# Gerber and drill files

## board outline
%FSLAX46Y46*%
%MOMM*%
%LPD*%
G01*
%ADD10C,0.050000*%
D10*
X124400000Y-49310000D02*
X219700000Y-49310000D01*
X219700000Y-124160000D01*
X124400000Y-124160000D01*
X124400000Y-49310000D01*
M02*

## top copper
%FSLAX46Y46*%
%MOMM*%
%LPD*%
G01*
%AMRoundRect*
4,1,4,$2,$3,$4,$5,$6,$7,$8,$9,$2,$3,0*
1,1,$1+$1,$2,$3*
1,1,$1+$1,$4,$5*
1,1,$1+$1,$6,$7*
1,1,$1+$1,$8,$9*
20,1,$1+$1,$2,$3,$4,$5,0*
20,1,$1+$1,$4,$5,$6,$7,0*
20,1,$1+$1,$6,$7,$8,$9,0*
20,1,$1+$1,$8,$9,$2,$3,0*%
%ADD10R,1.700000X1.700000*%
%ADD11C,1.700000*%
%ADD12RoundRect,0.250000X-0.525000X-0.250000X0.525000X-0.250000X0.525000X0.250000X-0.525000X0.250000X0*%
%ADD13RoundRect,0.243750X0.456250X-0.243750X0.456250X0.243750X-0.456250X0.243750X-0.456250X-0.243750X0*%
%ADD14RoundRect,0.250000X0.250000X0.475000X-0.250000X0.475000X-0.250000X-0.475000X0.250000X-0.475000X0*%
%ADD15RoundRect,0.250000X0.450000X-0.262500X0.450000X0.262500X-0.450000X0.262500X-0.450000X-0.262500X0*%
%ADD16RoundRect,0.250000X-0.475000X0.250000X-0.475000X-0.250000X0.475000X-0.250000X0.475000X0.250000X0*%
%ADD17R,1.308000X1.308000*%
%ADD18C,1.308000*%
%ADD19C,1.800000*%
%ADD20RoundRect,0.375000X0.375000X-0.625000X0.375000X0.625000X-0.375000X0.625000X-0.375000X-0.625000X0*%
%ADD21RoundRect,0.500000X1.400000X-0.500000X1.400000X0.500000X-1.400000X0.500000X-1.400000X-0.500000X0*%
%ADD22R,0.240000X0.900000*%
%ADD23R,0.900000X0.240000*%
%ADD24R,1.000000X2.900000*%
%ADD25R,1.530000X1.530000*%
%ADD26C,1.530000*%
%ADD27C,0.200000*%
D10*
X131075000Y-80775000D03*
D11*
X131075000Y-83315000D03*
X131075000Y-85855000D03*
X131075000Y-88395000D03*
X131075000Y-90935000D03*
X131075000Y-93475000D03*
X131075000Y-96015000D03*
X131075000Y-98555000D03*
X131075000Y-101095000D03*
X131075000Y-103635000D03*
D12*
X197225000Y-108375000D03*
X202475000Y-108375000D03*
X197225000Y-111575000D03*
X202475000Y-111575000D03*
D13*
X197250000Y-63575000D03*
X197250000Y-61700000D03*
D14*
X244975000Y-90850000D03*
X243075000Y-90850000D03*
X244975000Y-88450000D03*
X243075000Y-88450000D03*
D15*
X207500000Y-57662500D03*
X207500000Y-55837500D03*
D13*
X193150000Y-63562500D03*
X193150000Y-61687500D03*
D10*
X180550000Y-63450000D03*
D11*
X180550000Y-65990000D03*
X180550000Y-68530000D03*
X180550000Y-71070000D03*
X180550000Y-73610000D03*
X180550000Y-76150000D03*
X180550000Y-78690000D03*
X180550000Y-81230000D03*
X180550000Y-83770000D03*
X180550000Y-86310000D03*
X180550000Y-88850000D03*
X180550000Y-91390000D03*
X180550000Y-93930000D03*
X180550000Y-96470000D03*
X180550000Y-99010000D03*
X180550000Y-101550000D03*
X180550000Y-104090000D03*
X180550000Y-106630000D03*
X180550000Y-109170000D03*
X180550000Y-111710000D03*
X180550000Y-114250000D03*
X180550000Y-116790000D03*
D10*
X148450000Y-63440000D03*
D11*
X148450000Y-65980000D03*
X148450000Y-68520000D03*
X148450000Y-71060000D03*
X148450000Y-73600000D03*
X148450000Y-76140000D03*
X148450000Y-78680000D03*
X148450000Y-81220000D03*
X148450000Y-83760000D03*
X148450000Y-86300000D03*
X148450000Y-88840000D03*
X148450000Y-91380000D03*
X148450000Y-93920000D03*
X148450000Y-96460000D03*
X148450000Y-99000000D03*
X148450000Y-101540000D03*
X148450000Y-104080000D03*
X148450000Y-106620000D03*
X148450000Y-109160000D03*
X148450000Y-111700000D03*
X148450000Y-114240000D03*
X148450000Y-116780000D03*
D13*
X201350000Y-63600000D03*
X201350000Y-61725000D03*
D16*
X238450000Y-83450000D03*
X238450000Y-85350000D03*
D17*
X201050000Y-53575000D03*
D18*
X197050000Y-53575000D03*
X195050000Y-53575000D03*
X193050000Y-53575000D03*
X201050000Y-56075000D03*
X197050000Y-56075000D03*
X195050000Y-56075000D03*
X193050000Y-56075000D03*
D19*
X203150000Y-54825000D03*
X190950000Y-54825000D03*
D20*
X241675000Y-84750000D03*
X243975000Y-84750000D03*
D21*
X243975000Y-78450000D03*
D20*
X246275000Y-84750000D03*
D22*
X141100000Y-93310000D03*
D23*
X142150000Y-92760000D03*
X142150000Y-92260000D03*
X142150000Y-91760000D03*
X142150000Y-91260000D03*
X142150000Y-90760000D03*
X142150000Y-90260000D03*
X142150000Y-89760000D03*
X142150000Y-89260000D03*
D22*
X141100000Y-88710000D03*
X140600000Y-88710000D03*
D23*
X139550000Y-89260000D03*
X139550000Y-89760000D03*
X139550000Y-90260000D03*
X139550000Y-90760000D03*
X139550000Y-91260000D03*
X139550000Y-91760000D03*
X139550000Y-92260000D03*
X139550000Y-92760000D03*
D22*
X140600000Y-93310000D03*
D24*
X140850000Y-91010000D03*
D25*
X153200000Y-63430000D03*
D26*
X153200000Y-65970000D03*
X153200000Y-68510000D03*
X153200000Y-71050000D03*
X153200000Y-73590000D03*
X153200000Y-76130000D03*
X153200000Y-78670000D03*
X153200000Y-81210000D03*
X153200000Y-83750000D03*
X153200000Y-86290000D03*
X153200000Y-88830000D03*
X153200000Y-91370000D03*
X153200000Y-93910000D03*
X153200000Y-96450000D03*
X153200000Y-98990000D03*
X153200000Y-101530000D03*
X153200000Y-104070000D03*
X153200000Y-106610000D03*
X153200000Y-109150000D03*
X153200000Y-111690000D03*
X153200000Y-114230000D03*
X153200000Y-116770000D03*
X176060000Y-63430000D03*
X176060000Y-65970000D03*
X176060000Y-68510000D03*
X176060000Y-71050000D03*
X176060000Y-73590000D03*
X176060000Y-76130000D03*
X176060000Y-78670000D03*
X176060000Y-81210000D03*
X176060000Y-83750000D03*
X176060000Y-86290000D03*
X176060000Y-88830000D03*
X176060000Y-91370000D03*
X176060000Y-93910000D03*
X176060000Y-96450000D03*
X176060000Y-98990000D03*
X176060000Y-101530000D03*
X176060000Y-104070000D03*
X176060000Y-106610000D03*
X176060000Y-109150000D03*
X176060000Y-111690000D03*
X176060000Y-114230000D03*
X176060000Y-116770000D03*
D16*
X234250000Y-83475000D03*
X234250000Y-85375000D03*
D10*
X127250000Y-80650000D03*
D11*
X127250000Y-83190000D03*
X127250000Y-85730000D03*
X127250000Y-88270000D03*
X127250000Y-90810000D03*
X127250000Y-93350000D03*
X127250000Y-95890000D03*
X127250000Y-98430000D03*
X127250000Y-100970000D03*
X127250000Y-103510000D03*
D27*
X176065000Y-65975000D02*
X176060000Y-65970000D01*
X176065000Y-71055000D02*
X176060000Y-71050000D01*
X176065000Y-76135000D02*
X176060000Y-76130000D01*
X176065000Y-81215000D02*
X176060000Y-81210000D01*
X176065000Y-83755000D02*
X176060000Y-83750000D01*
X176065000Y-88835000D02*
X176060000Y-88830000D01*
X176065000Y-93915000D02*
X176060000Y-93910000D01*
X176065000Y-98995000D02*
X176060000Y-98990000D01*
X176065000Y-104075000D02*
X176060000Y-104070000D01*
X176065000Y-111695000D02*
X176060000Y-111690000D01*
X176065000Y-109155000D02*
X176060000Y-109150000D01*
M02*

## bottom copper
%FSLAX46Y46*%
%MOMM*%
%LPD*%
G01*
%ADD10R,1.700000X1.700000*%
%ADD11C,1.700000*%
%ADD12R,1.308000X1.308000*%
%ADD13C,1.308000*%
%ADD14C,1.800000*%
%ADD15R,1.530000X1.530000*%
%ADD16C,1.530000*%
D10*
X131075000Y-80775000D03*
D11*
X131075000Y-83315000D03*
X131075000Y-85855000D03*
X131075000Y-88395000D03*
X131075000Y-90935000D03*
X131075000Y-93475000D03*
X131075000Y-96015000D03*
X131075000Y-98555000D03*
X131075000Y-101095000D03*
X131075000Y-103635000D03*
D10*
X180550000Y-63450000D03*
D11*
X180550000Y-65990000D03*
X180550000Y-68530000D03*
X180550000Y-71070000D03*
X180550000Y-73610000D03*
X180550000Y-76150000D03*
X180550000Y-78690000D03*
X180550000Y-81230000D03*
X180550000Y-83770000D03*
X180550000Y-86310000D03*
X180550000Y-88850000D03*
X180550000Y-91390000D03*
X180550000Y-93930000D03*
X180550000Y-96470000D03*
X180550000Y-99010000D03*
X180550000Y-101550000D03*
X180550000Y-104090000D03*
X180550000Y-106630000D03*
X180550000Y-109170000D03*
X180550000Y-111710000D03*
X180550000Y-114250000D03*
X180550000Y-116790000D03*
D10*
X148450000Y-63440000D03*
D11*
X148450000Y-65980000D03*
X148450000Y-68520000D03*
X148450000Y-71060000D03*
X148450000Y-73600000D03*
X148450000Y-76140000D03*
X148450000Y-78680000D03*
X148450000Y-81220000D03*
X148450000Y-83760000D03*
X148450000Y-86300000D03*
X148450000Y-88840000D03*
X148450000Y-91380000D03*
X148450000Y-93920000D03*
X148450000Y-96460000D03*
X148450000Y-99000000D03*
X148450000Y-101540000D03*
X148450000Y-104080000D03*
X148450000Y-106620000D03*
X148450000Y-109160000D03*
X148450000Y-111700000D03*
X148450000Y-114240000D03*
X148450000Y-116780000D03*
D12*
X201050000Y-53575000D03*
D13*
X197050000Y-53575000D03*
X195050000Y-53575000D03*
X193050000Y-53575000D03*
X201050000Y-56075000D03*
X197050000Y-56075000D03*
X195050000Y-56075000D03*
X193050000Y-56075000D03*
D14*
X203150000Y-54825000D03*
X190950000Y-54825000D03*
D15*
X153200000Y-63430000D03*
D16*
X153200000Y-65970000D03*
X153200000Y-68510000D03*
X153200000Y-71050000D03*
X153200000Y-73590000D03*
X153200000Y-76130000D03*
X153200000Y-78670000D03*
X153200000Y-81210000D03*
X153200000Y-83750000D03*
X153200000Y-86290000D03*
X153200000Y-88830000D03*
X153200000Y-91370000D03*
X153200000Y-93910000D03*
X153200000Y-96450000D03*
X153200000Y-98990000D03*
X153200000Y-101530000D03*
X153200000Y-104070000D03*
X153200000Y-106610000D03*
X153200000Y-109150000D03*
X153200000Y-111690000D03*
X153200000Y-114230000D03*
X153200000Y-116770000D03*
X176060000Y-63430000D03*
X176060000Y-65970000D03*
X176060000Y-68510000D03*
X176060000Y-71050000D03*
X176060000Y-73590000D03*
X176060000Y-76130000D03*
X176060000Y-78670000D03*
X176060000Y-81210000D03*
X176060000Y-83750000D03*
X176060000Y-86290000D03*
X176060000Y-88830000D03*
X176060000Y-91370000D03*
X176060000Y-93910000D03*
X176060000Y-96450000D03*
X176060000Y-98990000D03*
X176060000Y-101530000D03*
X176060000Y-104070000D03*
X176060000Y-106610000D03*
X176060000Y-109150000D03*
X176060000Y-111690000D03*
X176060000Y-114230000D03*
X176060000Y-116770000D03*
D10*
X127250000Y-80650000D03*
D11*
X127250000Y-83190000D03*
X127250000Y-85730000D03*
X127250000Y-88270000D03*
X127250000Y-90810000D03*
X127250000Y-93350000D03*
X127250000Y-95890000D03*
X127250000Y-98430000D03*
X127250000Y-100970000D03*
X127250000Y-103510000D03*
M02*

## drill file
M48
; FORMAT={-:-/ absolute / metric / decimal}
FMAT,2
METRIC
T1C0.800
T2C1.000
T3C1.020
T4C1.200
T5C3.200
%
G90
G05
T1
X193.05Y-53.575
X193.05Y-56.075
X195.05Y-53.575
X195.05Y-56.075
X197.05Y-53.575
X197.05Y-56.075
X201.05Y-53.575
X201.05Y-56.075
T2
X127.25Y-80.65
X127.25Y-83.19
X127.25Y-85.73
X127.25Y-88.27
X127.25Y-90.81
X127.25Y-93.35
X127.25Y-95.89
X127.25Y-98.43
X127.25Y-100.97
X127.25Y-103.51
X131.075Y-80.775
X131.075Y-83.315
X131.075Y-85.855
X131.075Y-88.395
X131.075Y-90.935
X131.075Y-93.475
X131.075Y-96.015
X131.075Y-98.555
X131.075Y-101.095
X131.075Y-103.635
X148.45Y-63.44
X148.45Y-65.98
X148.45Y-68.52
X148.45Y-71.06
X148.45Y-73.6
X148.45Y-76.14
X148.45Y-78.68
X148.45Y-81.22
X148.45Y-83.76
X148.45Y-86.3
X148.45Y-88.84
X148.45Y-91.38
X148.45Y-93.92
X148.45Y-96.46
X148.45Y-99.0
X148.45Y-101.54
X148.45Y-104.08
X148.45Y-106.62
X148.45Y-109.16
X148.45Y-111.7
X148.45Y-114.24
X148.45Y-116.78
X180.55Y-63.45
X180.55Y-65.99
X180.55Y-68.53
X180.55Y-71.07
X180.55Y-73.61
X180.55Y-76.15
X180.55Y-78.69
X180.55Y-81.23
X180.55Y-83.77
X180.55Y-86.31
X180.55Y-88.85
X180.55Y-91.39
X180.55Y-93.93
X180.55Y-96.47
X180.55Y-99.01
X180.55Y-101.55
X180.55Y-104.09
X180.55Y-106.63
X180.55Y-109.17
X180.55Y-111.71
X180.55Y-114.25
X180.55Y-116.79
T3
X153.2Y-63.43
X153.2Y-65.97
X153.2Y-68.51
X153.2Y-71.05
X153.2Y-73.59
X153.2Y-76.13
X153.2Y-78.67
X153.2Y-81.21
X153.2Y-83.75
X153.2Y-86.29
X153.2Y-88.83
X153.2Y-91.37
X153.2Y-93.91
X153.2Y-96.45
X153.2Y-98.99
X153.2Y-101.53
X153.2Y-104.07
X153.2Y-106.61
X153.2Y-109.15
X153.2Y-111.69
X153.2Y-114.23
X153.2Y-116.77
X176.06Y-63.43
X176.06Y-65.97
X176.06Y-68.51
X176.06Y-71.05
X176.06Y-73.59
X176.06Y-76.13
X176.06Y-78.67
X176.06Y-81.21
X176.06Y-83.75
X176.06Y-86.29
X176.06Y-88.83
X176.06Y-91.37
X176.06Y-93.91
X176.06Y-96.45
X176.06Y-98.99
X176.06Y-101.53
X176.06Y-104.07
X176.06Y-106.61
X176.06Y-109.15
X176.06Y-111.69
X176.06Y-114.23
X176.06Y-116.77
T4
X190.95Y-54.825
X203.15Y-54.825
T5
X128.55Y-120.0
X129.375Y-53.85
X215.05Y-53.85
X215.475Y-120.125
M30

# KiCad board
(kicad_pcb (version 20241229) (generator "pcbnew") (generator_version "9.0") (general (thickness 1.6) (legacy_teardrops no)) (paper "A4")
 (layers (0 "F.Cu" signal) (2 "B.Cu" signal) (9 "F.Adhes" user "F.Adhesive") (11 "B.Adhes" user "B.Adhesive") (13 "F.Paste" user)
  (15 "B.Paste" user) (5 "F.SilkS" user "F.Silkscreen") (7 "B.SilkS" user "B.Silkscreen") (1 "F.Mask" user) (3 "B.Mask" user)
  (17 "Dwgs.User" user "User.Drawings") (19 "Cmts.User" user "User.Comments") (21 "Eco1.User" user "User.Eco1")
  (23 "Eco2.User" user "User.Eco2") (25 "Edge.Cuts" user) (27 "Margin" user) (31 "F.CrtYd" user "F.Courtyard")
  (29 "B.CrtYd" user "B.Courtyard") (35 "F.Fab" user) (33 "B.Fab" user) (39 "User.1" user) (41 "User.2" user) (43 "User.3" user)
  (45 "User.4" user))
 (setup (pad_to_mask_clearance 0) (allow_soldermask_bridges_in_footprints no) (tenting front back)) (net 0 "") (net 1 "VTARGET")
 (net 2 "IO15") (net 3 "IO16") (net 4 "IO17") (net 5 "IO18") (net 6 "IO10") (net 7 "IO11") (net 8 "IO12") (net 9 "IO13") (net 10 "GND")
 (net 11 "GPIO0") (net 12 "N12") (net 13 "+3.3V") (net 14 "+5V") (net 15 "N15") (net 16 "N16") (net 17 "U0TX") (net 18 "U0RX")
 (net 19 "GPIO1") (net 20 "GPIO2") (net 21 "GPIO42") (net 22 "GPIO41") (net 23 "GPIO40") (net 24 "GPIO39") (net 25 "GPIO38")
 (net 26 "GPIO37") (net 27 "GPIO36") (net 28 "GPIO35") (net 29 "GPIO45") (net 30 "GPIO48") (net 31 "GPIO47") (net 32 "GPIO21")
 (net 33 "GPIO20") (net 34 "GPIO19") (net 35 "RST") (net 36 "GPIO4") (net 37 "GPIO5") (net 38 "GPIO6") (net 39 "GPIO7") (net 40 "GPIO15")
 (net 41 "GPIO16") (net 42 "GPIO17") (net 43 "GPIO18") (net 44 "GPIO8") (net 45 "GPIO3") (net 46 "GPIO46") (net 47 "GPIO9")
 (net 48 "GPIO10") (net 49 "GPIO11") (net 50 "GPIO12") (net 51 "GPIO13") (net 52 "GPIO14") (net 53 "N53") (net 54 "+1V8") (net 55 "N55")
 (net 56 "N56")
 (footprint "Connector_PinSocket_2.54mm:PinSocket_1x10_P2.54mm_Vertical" (layer "F.Cu") (at 131.075 80.775)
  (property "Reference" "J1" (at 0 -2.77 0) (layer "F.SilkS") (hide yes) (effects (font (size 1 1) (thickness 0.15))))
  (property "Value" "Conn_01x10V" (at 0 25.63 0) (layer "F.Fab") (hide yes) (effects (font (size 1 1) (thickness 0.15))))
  (pad "1" thru_hole rect (at 0 0) (size 1.7 1.7) (drill 1) (layers "*.Cu" "*.Mask") (remove_unused_layers no) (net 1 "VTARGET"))
  (pad "2" thru_hole circle (at 0 2.54) (size 1.7 1.7) (drill 1) (layers "*.Cu" "*.Mask") (remove_unused_layers no) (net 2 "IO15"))
  (pad "3" thru_hole circle (at 0 5.08) (size 1.7 1.7) (drill 1) (layers "*.Cu" "*.Mask") (remove_unused_layers no) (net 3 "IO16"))
  (pad "4" thru_hole circle (at 0 7.62) (size 1.7 1.7) (drill 1) (layers "*.Cu" "*.Mask") (remove_unused_layers no) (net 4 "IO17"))
  (pad "5" thru_hole circle (at 0 10.16) (size 1.7 1.7) (drill 1) (layers "*.Cu" "*.Mask") (remove_unused_layers no) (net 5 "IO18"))
  (pad "6" thru_hole circle (at 0 12.7) (size 1.7 1.7) (drill 1) (layers "*.Cu" "*.Mask") (remove_unused_layers no) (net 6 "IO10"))
  (pad "7" thru_hole circle (at 0 15.24) (size 1.7 1.7) (drill 1) (layers "*.Cu" "*.Mask") (remove_unused_layers no) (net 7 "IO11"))
  (pad "8" thru_hole circle (at 0 17.78) (size 1.7 1.7) (drill 1) (layers "*.Cu" "*.Mask") (remove_unused_layers no) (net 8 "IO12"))
  (pad "9" thru_hole circle (at 0 20.32) (size 1.7 1.7) (drill 1) (layers "*.Cu" "*.Mask") (remove_unused_layers no) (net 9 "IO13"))
  (pad "10" thru_hole circle (at 0 22.86) (size 1.7 1.7) (drill 1) (layers "*.Cu" "*.Mask") (remove_unused_layers no) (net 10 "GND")))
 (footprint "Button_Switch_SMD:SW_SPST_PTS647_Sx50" (layer "F.Cu") (at 199.85 109.975)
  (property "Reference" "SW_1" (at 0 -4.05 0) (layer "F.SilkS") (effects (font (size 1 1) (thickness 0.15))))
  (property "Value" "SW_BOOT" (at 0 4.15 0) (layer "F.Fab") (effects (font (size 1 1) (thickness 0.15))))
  (pad "1" smd roundrect (at -2.625 -1.6) (size 1.55 1) (layers "F.Cu" "F.Mask" "F.Paste") (roundrect_rratio 0.25) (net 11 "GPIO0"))
  (pad "1" smd roundrect (at 2.625 -1.6) (size 1.55 1) (layers "F.Cu" "F.Mask" "F.Paste") (roundrect_rratio 0.25) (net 11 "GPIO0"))
  (pad "2" smd roundrect (at -2.625 1.6) (size 1.55 1) (layers "F.Cu" "F.Mask" "F.Paste") (roundrect_rratio 0.25) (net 10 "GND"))
  (pad "2" smd roundrect (at 2.625 1.6) (size 1.55 1) (layers "F.Cu" "F.Mask" "F.Paste") (roundrect_rratio 0.25) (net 10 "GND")))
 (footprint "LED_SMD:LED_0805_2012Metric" (layer "F.Cu") (at 197.25 62.6375 90)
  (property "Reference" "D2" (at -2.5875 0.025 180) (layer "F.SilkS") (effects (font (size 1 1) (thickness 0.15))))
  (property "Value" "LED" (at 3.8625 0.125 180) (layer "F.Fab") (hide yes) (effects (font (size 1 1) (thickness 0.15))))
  (pad "1" smd roundrect (at -0.9375 0 90) (size 0.975 1.4) (layers "F.Cu" "F.Mask" "F.Paste") (roundrect_rratio 0.25) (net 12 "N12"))
  (pad "2" smd roundrect (at 0.9375 0 90) (size 0.975 1.4) (layers "F.Cu" "F.Mask" "F.Paste") (roundrect_rratio 0.25) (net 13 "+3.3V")))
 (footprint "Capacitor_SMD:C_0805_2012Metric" (layer "F.Cu") (at 244.025 90.85 180)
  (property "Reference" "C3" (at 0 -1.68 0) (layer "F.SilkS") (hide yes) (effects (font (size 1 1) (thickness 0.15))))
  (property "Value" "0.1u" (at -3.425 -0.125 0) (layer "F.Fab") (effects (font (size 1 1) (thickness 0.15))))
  (pad "1" smd roundrect (at -0.95 0 180) (size 1 1.45) (layers "F.Cu" "F.Mask" "F.Paste") (roundrect_rratio 0.25) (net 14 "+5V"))
  (pad "2" smd roundrect (at 0.95 0 180) (size 1 1.45) (layers "F.Cu" "F.Mask" "F.Paste") (roundrect_rratio 0.25) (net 10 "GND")))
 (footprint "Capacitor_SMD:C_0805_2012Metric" (layer "F.Cu") (at 244.025 88.45 180)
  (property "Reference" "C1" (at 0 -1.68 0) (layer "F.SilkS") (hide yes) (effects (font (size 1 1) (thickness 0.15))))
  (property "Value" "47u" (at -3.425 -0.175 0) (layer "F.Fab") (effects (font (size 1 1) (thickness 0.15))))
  (pad "1" smd roundrect (at -0.95 0 180) (size 1 1.45) (layers "F.Cu" "F.Mask" "F.Paste") (roundrect_rratio 0.25) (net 14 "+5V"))
  (pad "2" smd roundrect (at 0.95 0 180) (size 1 1.45) (layers "F.Cu" "F.Mask" "F.Paste") (roundrect_rratio 0.25) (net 10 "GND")))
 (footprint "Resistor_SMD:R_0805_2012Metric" (layer "F.Cu") (at 207.5 56.75 90)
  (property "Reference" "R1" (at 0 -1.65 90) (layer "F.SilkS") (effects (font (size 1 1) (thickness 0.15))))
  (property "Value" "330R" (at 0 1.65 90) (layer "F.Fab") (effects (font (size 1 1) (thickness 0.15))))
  (pad "1" smd roundrect (at -0.9125 0 90) (size 1.025 1.4) (layers "F.Cu" "F.Mask" "F.Paste") (roundrect_rratio 0.243902) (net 10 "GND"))
  (pad "2" smd roundrect (at 0.9125 0 90) (size 1.025 1.4) (layers "F.Cu" "F.Mask" "F.Paste") (roundrect_rratio 0.243902) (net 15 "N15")))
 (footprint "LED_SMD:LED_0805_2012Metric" (layer "F.Cu") (at 193.15 62.625 90)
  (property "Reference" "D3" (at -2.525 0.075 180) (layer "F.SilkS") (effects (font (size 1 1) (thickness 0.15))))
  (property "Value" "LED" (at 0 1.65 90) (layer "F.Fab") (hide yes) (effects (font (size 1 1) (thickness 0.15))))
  (pad "1" smd roundrect (at -0.9375 0 90) (size 0.975 1.4) (layers "F.Cu" "F.Mask" "F.Paste") (roundrect_rratio 0.25) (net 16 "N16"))
  (pad "2" smd roundrect (at 0.9375 0 90) (size 0.975 1.4) (layers "F.Cu" "F.Mask" "F.Paste") (roundrect_rratio 0.25) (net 13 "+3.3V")))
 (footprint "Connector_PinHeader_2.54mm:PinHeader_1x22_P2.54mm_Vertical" (layer "F.Cu") (at 180.55 63.45)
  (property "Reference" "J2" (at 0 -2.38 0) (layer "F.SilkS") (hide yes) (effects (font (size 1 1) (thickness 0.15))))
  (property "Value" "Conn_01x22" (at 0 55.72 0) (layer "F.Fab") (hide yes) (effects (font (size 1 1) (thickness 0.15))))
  (pad "1" thru_hole rect (at 0 0) (size 1.7 1.7) (drill 1) (layers "*.Cu" "*.Mask") (remove_unused_layers no) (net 10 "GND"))
  (pad "2" thru_hole circle (at 0 2.54) (size 1.7 1.7) (drill 1) (layers "*.Cu" "*.Mask") (remove_unused_layers no) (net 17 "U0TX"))
  (pad "3" thru_hole circle (at 0 5.08) (size 1.7 1.7) (drill 1) (layers "*.Cu" "*.Mask") (remove_unused_layers no) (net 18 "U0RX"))
  (pad "4" thru_hole circle (at 0 7.62) (size 1.7 1.7) (drill 1) (layers "*.Cu" "*.Mask") (remove_unused_layers no) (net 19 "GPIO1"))
  (pad "5" thru_hole circle (at 0 10.16) (size 1.7 1.7) (drill 1) (layers "*.Cu" "*.Mask") (remove_unused_layers no) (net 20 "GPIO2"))
  (pad "6" thru_hole circle (at 0 12.7) (size 1.7 1.7) (drill 1) (layers "*.Cu" "*.Mask") (remove_unused_layers no) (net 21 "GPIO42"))
  (pad "7" thru_hole circle (at 0 15.24) (size 1.7 1.7) (drill 1) (layers "*.Cu" "*.Mask") (remove_unused_layers no) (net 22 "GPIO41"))
  (pad "8" thru_hole circle (at 0 17.78) (size 1.7 1.7) (drill 1) (layers "*.Cu" "*.Mask") (remove_unused_layers no) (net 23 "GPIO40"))
  (pad "9" thru_hole circle (at 0 20.32) (size 1.7 1.7) (drill 1) (layers "*.Cu" "*.Mask") (remove_unused_layers no) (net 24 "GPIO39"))
  (pad "10" thru_hole circle (at 0 22.86) (size 1.7 1.7) (drill 1) (layers "*.Cu" "*.Mask") (remove_unused_layers no) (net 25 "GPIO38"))
  (pad "11" thru_hole circle (at 0 25.4) (size 1.7 1.7) (drill 1) (layers "*.Cu" "*.Mask") (remove_unused_layers no) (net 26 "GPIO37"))
  (pad "12" thru_hole circle (at 0 27.94) (size 1.7 1.7) (drill 1) (layers "*.Cu" "*.Mask") (remove_unused_layers no) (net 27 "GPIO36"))
  (pad "13" thru_hole circle (at 0 30.48) (size 1.7 1.7) (drill 1) (layers "*.Cu" "*.Mask") (remove_unused_layers no) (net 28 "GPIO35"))
  (pad "14" thru_hole circle (at 0 33.02) (size 1.7 1.7) (drill 1) (layers "*.Cu" "*.Mask") (remove_unused_layers no) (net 11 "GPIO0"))
  (pad "15" thru_hole circle (at 0 35.56) (size 1.7 1.7) (drill 1) (layers "*.Cu" "*.Mask") (remove_unused_layers no) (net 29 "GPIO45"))
  (pad "16" thru_hole circle (at 0 38.1) (size 1.7 1.7) (drill 1) (layers "*.Cu" "*.Mask") (remove_unused_layers no) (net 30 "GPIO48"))
  (pad "17" thru_hole circle (at 0 40.64) (size 1.7 1.7) (drill 1) (layers "*.Cu" "*.Mask") (remove_unused_layers no) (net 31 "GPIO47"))
  (pad "18" thru_hole circle (at 0 43.18) (size 1.7 1.7) (drill 1) (layers "*.Cu" "*.Mask") (remove_unused_layers no) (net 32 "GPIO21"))
  (pad "19" thru_hole circle (at 0 45.72) (size 1.7 1.7) (drill 1) (layers "*.Cu" "*.Mask") (remove_unused_layers no) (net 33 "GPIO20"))
  (pad "20" thru_hole circle (at 0 48.26) (size 1.7 1.7) (drill 1) (layers "*.Cu" "*.Mask") (remove_unused_layers no) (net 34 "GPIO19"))
  (pad "21" thru_hole circle (at 0 50.8) (size 1.7 1.7) (drill 1) (layers "*.Cu" "*.Mask") (remove_unused_layers no) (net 10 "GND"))
  (pad "22" thru_hole circle (at 0 53.34) (size 1.7 1.7) (drill 1) (layers "*.Cu" "*.Mask") (remove_unused_layers no) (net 10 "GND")))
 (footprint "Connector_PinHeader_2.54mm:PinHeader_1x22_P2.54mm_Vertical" (layer "F.Cu") (at 148.45 63.44)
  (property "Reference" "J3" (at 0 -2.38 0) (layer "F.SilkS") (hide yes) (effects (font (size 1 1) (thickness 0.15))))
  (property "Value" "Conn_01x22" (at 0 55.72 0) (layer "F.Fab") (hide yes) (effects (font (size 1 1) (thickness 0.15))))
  (pad "1" thru_hole rect (at 0 0) (size 1.7 1.7) (drill 1) (layers "*.Cu" "*.Mask") (remove_unused_layers no) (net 13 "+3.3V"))
  (pad "2" thru_hole circle (at 0 2.54) (size 1.7 1.7) (drill 1) (layers "*.Cu" "*.Mask") (remove_unused_layers no) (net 13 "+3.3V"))
  (pad "3" thru_hole circle (at 0 5.08) (size 1.7 1.7) (drill 1) (layers "*.Cu" "*.Mask") (remove_unused_layers no) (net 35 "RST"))
  (pad "4" thru_hole circle (at 0 7.62) (size 1.7 1.7) (drill 1) (layers "*.Cu" "*.Mask") (remove_unused_layers no) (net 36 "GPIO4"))
  (pad "5" thru_hole circle (at 0 10.16) (size 1.7 1.7) (drill 1) (layers "*.Cu" "*.Mask") (remove_unused_layers no) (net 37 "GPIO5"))
  (pad "6" thru_hole circle (at 0 12.7) (size 1.7 1.7) (drill 1) (layers "*.Cu" "*.Mask") (remove_unused_layers no) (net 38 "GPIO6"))
  (pad "7" thru_hole circle (at 0 15.24) (size 1.7 1.7) (drill 1) (layers "*.Cu" "*.Mask") (remove_unused_layers no) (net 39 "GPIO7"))
  (pad "8" thru_hole circle (at 0 17.78) (size 1.7 1.7) (drill 1) (layers "*.Cu" "*.Mask") (remove_unused_layers no) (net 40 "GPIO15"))
  (pad "9" thru_hole circle (at 0 20.32) (size 1.7 1.7) (drill 1) (layers "*.Cu" "*.Mask") (remove_unused_layers no) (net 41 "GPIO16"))
  (pad "10" thru_hole circle (at 0 22.86) (size 1.7 1.7) (drill 1) (layers "*.Cu" "*.Mask") (remove_unused_layers no) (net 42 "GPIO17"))
  (pad "11" thru_hole circle (at 0 25.4) (size 1.7 1.7) (drill 1) (layers "*.Cu" "*.Mask") (remove_unused_layers no) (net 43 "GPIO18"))
  (pad "12" thru_hole circle (at 0 27.94) (size 1.7 1.7) (drill 1) (layers "*.Cu" "*.Mask") (remove_unused_layers no) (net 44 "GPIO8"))
  (pad "13" thru_hole circle (at 0 30.48) (size 1.7 1.7) (drill 1) (layers "*.Cu" "*.Mask") (remove_unused_layers no) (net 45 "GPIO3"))
  (pad "14" thru_hole circle (at 0 33.02) (size 1.7 1.7) (drill 1) (layers "*.Cu" "*.Mask") (remove_unused_layers no) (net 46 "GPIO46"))
  (pad "15" thru_hole circle (at 0 35.56) (size 1.7 1.7) (drill 1) (layers "*.Cu" "*.Mask") (remove_unused_layers no) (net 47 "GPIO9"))
  (pad "16" thru_hole circle (at 0 38.1) (size 1.7 1.7) (drill 1) (layers "*.Cu" "*.Mask") (remove_unused_layers no) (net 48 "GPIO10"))
  (pad "17" thru_hole circle (at 0 40.64) (size 1.7 1.7) (drill 1) (layers "*.Cu" "*.Mask") (remove_unused_layers no) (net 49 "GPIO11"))
  (pad "18" thru_hole circle (at 0 43.18) (size 1.7 1.7) (drill 1) (layers "*.Cu" "*.Mask") (remove_unused_layers no) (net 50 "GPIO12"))
  (pad "19" thru_hole circle (at 0 45.72) (size 1.7 1.7) (drill 1) (layers "*.Cu" "*.Mask") (remove_unused_layers no) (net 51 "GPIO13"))
  (pad "20" thru_hole circle (at 0 48.26) (size 1.7 1.7) (drill 1) (layers "*.Cu" "*.Mask") (remove_unused_layers no) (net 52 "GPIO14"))
  (pad "21" thru_hole circle (at 0 50.8) (size 1.7 1.7) (drill 1) (layers "*.Cu" "*.Mask") (remove_unused_layers no) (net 14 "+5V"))
  (pad "22" thru_hole circle (at 0 53.34) (size 1.7 1.7) (drill 1) (layers "*.Cu" "*.Mask") (remove_unused_layers no) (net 10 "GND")))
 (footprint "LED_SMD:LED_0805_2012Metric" (layer "F.Cu") (at 201.35 62.6625 90)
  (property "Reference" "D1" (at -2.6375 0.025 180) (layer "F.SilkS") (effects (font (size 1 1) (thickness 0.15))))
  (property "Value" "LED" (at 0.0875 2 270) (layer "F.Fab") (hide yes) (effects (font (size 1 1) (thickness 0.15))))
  (pad "1" smd roundrect (at -0.9375 0 90) (size 0.975 1.4) (layers "F.Cu" "F.Mask" "F.Paste") (roundrect_rratio 0.25) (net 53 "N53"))
  (pad "2" smd roundrect (at 0.9375 0 90) (size 0.975 1.4) (layers "F.Cu" "F.Mask" "F.Paste") (roundrect_rratio 0.25) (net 13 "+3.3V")))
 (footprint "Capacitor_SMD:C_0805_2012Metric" (layer "F.Cu") (at 238.45 84.4 -90)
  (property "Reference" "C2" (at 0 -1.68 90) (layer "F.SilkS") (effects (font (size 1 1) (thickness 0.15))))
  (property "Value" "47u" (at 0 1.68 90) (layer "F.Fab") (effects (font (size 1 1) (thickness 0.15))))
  (pad "1" smd roundrect (at -0.95 0 270) (size 1 1.45) (layers "F.Cu" "F.Mask" "F.Paste") (roundrect_rratio 0.25) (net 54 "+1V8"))
  (pad "2" smd roundrect (at 0.95 0 270) (size 1 1.45) (layers "F.Cu" "F.Mask" "F.Paste") (roundrect_rratio 0.25) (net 10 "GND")))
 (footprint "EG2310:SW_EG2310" (layer "F.Cu") (at 197.05 54.825 180)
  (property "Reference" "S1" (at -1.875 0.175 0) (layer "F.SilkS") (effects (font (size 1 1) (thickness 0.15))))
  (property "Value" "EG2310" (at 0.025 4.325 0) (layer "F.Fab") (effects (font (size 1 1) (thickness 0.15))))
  (pad "1" thru_hole rect (at -4 1.25 180) (size 1.308 1.308) (drill 0.8) (layers "*.Cu" "*.Mask") (remove_unused_layers no) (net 54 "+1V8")
   (solder_mask_margin 0.102))
  (pad "2" thru_hole circle (at 0 1.25 180) (size 1.308 1.308) (drill 0.8) (layers "*.Cu" "*.Mask") (remove_unused_layers no)
   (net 1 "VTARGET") (solder_mask_margin 0.102))
  (pad "3" thru_hole circle (at 2 1.25 180) (size 1.308 1.308) (drill 0.8) (layers "*.Cu" "*.Mask") (remove_unused_layers no)
   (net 13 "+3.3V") (solder_mask_margin 0.102))
  (pad "4" thru_hole circle (at 4 1.25 180) (size 1.308 1.308) (drill 0.8) (layers "*.Cu" "*.Mask") (remove_unused_layers no) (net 14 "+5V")
   (solder_mask_margin 0.102))
  (pad "5" thru_hole circle (at -4 -1.25 180) (size 1.308 1.308) (drill 0.8) (layers "*.Cu" "*.Mask") (remove_unused_layers no)
   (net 53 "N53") (solder_mask_margin 0.102))
  (pad "6" thru_hole circle (at 0 -1.25 180) (size 1.308 1.308) (drill 0.8) (layers "*.Cu" "*.Mask") (remove_unused_layers no)
   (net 15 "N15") (solder_mask_margin 0.102))
  (pad "7" thru_hole circle (at 2 -1.25 180) (size 1.308 1.308) (drill 0.8) (layers "*.Cu" "*.Mask") (remove_unused_layers no)
   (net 12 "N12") (solder_mask_margin 0.102))
  (pad "8" thru_hole circle (at 4 -1.25 180) (size 1.308 1.308) (drill 0.8) (layers "*.Cu" "*.Mask") (remove_unused_layers no)
   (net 16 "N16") (solder_mask_margin 0.102))
  (pad "SH1" thru_hole circle (at -6.1 0 180) (size 1.8 1.8) (drill 1.2) (layers "*.Cu" "*.Mask") (remove_unused_layers no)
   (solder_mask_margin 0.102))
  (pad "SH2" thru_hole circle (at 6.1 0 180) (size 1.8 1.8) (drill 1.2) (layers "*.Cu" "*.Mask") (remove_unused_layers no)
   (solder_mask_margin 0.102)))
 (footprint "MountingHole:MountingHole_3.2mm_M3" (layer "F.Cu") (at 215.475 120.125)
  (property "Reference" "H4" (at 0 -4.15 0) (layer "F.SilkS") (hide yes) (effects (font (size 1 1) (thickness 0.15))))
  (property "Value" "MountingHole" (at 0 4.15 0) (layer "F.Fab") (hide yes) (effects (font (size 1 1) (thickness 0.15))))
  (pad "" np_thru_hole circle (at 0 0) (size 3.2 3.2) (drill 3.2) (layers "*.Cu" "*.Mask")))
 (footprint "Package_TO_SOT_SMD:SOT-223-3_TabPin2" (layer "F.Cu") (at 243.975 81.6 90)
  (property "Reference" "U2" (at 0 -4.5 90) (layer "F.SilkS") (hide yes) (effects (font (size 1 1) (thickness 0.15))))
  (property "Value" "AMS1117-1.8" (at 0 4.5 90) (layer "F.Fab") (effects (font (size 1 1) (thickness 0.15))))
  (pad "1" smd roundrect (at -3.15 -2.3 90) (size 2 1.5) (layers "F.Cu" "F.Mask" "F.Paste") (roundrect_rratio 0.25) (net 10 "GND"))
  (pad "2" smd roundrect (at -3.15 0 90) (size 2 1.5) (layers "F.Cu" "F.Mask" "F.Paste") (roundrect_rratio 0.25) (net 54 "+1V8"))
  (pad "2" smd roundrect (at 3.15 0 90) (size 2 3.8) (layers "F.Cu" "F.Mask" "F.Paste") (roundrect_rratio 0.25) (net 54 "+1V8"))
  (pad "3" smd roundrect (at -3.15 2.3 90) (size 2 1.5) (layers "F.Cu" "F.Mask" "F.Paste") (roundrect_rratio 0.25) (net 14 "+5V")))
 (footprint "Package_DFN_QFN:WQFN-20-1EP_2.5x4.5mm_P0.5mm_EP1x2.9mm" (layer "F.Cu") (at 140.85 91.01 180)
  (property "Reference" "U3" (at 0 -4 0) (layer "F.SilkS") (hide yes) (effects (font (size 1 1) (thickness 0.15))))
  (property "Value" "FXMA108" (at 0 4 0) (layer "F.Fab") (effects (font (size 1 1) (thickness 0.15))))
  (pad "" smd rect (at 0 -0.95 90) (size 0.8 0.8) (layers "F.Paste"))
  (pad "" smd rect (at 0 0 90) (size 0.8 0.8) (layers "F.Paste"))
  (pad "" smd rect (at 0 0.95 90) (size 0.8 0.8) (layers "F.Paste"))
  (pad "1" smd rect (at -0.25 -2.3 90) (size 0.9 0.24) (layers "F.Cu" "F.Mask" "F.Paste") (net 13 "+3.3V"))
  (pad "2" smd rect (at -1.3 -1.75 180) (size 0.9 0.24) (layers "F.Cu" "F.Mask" "F.Paste") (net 51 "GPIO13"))
  (pad "3" smd rect (at -1.3 -1.25 180) (size 0.9 0.24) (layers "F.Cu" "F.Mask" "F.Paste") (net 50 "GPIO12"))
  (pad "4" smd rect (at -1.3 -0.75 180) (size 0.9 0.24) (layers "F.Cu" "F.Mask" "F.Paste") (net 49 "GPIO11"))
  (pad "5" smd rect (at -1.3 -0.25 180) (size 0.9 0.24) (layers "F.Cu" "F.Mask" "F.Paste") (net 48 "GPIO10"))
  (pad "6" smd rect (at -1.3 0.25 180) (size 0.9 0.24) (layers "F.Cu" "F.Mask" "F.Paste") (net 43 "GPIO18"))
  (pad "7" smd rect (at -1.3 0.75 180) (size 0.9 0.24) (layers "F.Cu" "F.Mask" "F.Paste") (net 42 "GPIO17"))
  (pad "8" smd rect (at -1.3 1.25 180) (size 0.9 0.24) (layers "F.Cu" "F.Mask" "F.Paste") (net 41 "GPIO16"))
  (pad "9" smd rect (at -1.3 1.75 180) (size 0.9 0.24) (layers "F.Cu" "F.Mask" "F.Paste") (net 40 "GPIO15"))
  (pad "10" smd rect (at -0.25 2.3 90) (size 0.9 0.24) (layers "F.Cu" "F.Mask" "F.Paste") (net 10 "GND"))
  (pad "11" smd rect (at 0.25 2.3 90) (size 0.9 0.24) (layers "F.Cu" "F.Mask" "F.Paste") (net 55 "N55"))
  (pad "12" smd rect (at 1.3 1.75 180) (size 0.9 0.24) (layers "F.Cu" "F.Mask" "F.Paste") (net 2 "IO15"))
  (pad "13" smd rect (at 1.3 1.25 180) (size 0.9 0.24) (layers "F.Cu" "F.Mask" "F.Paste") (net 3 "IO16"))
  (pad "14" smd rect (at 1.3 0.75 180) (size 0.9 0.24) (layers "F.Cu" "F.Mask" "F.Paste") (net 4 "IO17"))
  (pad "15" smd rect (at 1.3 0.25 180) (size 0.9 0.24) (layers "F.Cu" "F.Mask" "F.Paste") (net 5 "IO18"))
  (pad "16" smd rect (at 1.3 -0.25 180) (size 0.9 0.24) (layers "F.Cu" "F.Mask" "F.Paste") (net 6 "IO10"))
  (pad "17" smd rect (at 1.3 -0.75 180) (size 0.9 0.24) (layers "F.Cu" "F.Mask" "F.Paste") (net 7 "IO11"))
  (pad "18" smd rect (at 1.3 -1.25 180) (size 0.9 0.24) (layers "F.Cu" "F.Mask" "F.Paste") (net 8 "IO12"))
  (pad "19" smd rect (at 1.3 -1.75 180) (size 0.9 0.24) (layers "F.Cu" "F.Mask" "F.Paste") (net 9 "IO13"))
  (pad "20" smd rect (at 0.25 -2.3 90) (size 0.9 0.24) (layers "F.Cu" "F.Mask" "F.Paste") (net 1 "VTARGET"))
  (pad "21" smd rect (at 0 0 90) (size 2.9 1) (layers "F.Cu" "F.Mask") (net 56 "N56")))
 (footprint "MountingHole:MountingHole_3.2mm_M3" (layer "F.Cu") (at 129.375 53.85)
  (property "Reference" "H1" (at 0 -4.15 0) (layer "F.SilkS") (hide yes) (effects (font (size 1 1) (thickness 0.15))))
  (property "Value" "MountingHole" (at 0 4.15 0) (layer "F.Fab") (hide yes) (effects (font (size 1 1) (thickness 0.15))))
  (pad "" np_thru_hole circle (at 0 0) (size 3.2 3.2) (drill 3.2) (layers "*.Cu" "*.Mask")))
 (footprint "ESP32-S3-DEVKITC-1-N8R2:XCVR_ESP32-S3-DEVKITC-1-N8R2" (layer "F.Cu") (at 164.63 93.4)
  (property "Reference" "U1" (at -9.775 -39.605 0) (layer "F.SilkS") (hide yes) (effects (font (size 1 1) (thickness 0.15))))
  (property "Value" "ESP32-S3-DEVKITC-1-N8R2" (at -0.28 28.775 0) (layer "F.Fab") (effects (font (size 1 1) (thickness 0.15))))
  (pad "J1_1" thru_hole rect (at -11.43 -29.97) (size 1.53 1.53) (drill 1.02) (layers "*.Cu" "*.Mask") (remove_unused_layers no)
   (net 13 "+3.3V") (solder_mask_margin 0.102))
  (pad "J1_2" thru_hole circle (at -11.43 -27.43) (size 1.53 1.53) (drill 1.02) (layers "*.Cu" "*.Mask") (remove_unused_layers no)
   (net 13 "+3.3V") (solder_mask_margin 0.102))
  (pad "J1_3" thru_hole circle (at -11.43 -24.89) (size 1.53 1.53) (drill 1.02) (layers "*.Cu" "*.Mask") (remove_unused_layers no)
   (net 35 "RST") (solder_mask_margin 0.102))
  (pad "J1_4" thru_hole circle (at -11.43 -22.35) (size 1.53 1.53) (drill 1.02) (layers "*.Cu" "*.Mask") (remove_unused_layers no)
   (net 36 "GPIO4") (solder_mask_margin 0.102))
  (pad "J1_5" thru_hole circle (at -11.43 -19.81) (size 1.53 1.53) (drill 1.02) (layers "*.Cu" "*.Mask") (remove_unused_layers no)
   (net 37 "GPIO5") (solder_mask_margin 0.102))
  (pad "J1_6" thru_hole circle (at -11.43 -17.27) (size 1.53 1.53) (drill 1.02) (layers "*.Cu" "*.Mask") (remove_unused_layers no)
   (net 38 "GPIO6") (solder_mask_margin 0.102))
  (pad "J1_7" thru_hole circle (at -11.43 -14.73) (size 1.53 1.53) (drill 1.02) (layers "*.Cu" "*.Mask") (remove_unused_layers no)
   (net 39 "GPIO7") (solder_mask_margin 0.102))
  (pad "J1_8" thru_hole circle (at -11.43 -12.19) (size 1.53 1.53) (drill 1.02) (layers "*.Cu" "*.Mask") (remove_unused_layers no)
   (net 40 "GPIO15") (solder_mask_margin 0.102))
  (pad "J1_9" thru_hole circle (at -11.43 -9.65) (size 1.53 1.53) (drill 1.02) (layers "*.Cu" "*.Mask") (remove_unused_layers no)
   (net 41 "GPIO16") (solder_mask_margin 0.102))
  (pad "J1_10" thru_hole circle (at -11.43 -7.11) (size 1.53 1.53) (drill 1.02) (layers "*.Cu" "*.Mask") (remove_unused_layers no)
   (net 42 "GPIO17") (solder_mask_margin 0.102))
  (pad "J1_11" thru_hole circle (at -11.43 -4.57) (size 1.53 1.53) (drill 1.02) (layers "*.Cu" "*.Mask") (remove_unused_layers no)
   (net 43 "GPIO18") (solder_mask_margin 0.102))
  (pad "J1_12" thru_hole circle (at -11.43 -2.03) (size 1.53 1.53) (drill 1.02) (layers "*.Cu" "*.Mask") (remove_unused_layers no)
   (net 44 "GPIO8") (solder_mask_margin 0.102))
  (pad "J1_13" thru_hole circle (at -11.43 0.51) (size 1.53 1.53) (drill 1.02) (layers "*.Cu" "*.Mask") (remove_unused_layers no)
   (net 45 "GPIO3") (solder_mask_margin 0.102))
  (pad "J1_14" thru_hole circle (at -11.43 3.05) (size 1.53 1.53) (drill 1.02) (layers "*.Cu" "*.Mask") (remove_unused_layers no)
   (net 46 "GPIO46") (solder_mask_margin 0.102))
  (pad "J1_15" thru_hole circle (at -11.43 5.59) (size 1.53 1.53) (drill 1.02) (layers "*.Cu" "*.Mask") (remove_unused_layers no)
   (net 47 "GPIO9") (solder_mask_margin 0.102))
  (pad "J1_16" thru_hole circle (at -11.43 8.13) (size 1.53 1.53) (drill 1.02) (layers "*.Cu" "*.Mask") (remove_unused_layers no)
   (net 48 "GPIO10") (solder_mask_margin 0.102))
  (pad "J1_17" thru_hole circle (at -11.43 10.67) (size 1.53 1.53) (drill 1.02) (layers "*.Cu" "*.Mask") (remove_unused_layers no)
   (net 49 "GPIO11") (solder_mask_margin 0.102))
  (pad "J1_18" thru_hole circle (at -11.43 13.21) (size 1.53 1.53) (drill 1.02) (layers "*.Cu" "*.Mask") (remove_unused_layers no)
   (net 50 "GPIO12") (solder_mask_margin 0.102))
  (pad "J1_19" thru_hole circle (at -11.43 15.75) (size 1.53 1.53) (drill 1.02) (layers "*.Cu" "*.Mask") (remove_unused_layers no)
   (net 51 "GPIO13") (solder_mask_margin 0.102))
  (pad "J1_20" thru_hole circle (at -11.43 18.29) (size 1.53 1.53) (drill 1.02) (layers "*.Cu" "*.Mask") (remove_unused_layers no)
   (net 52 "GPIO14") (solder_mask_margin 0.102))
  (pad "J1_21" thru_hole circle (at -11.43 20.83) (size 1.53 1.53) (drill 1.02) (layers "*.Cu" "*.Mask") (remove_unused_layers no)
   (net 14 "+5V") (solder_mask_margin 0.102))
  (pad "J1_22" thru_hole circle (at -11.43 23.37) (size 1.53 1.53) (drill 1.02) (layers "*.Cu" "*.Mask") (remove_unused_layers no)
   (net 10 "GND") (solder_mask_margin 0.102))
  (pad "J3_1" thru_hole circle (at 11.43 -29.97) (size 1.53 1.53) (drill 1.02) (layers "*.Cu" "*.Mask") (remove_unused_layers no)
   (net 10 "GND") (solder_mask_margin 0.102))
  (pad "J3_2" thru_hole circle (at 11.43 -27.43) (size 1.53 1.53) (drill 1.02) (layers "*.Cu" "*.Mask") (remove_unused_layers no)
   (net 17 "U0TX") (solder_mask_margin 0.102))
  (pad "J3_3" thru_hole circle (at 11.43 -24.89) (size 1.53 1.53) (drill 1.02) (layers "*.Cu" "*.Mask") (remove_unused_layers no)
   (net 18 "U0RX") (solder_mask_margin 0.102))
  (pad "J3_4" thru_hole circle (at 11.43 -22.35) (size 1.53 1.53) (drill 1.02) (layers "*.Cu" "*.Mask") (remove_unused_layers no)
   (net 19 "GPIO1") (solder_mask_margin 0.102))
  (pad "J3_5" thru_hole circle (at 11.43 -19.81) (size 1.53 1.53) (drill 1.02) (layers "*.Cu" "*.Mask") (remove_unused_layers no)
   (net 20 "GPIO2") (solder_mask_margin 0.102))
  (pad "J3_6" thru_hole circle (at 11.43 -17.27) (size 1.53 1.53) (drill 1.02) (layers "*.Cu" "*.Mask") (remove_unused_layers no)
   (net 21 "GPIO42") (solder_mask_margin 0.102))
  (pad "J3_7" thru_hole circle (at 11.43 -14.73) (size 1.53 1.53) (drill 1.02) (layers "*.Cu" "*.Mask") (remove_unused_layers no)
   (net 22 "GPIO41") (solder_mask_margin 0.102))
  (pad "J3_8" thru_hole circle (at 11.43 -12.19) (size 1.53 1.53) (drill 1.02) (layers "*.Cu" "*.Mask") (remove_unused_layers no)
   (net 23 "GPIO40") (solder_mask_margin 0.102))
  (pad "J3_9" thru_hole circle (at 11.43 -9.65) (size 1.53 1.53) (drill 1.02) (layers "*.Cu" "*.Mask") (remove_unused_layers no)
   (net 24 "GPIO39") (solder_mask_margin 0.102))
  (pad "J3_10" thru_hole circle (at 11.43 -7.11) (size 1.53 1.53) (drill 1.02) (layers "*.Cu" "*.Mask") (remove_unused_layers no)
   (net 25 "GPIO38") (solder_mask_margin 0.102))
  (pad "J3_11" thru_hole circle (at 11.43 -4.57) (size 1.53 1.53) (drill 1.02) (layers "*.Cu" "*.Mask") (remove_unused_layers no)
   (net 26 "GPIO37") (solder_mask_margin 0.102))
  (pad "J3_12" thru_hole circle (at 11.43 -2.03) (size 1.53 1.53) (drill 1.02) (layers "*.Cu" "*.Mask") (remove_unused_layers no)
   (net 27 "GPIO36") (solder_mask_margin 0.102))
  (pad "J3_13" thru_hole circle (at 11.43 0.51) (size 1.53 1.53) (drill 1.02) (layers "*.Cu" "*.Mask") (remove_unused_layers no)
   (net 28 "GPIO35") (solder_mask_margin 0.102))
  (pad "J3_14" thru_hole circle (at 11.43 3.05) (size 1.53 1.53) (drill 1.02) (layers "*.Cu" "*.Mask") (remove_unused_layers no)
   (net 11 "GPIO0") (solder_mask_margin 0.102))
  (pad "J3_15" thru_hole circle (at 11.43 5.59) (size 1.53 1.53) (drill 1.02) (layers "*.Cu" "*.Mask") (remove_unused_layers no)
   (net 29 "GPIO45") (solder_mask_margin 0.102))
  (pad "J3_16" thru_hole circle (at 11.43 8.13) (size 1.53 1.53) (drill 1.02) (layers "*.Cu" "*.Mask") (remove_unused_layers no)
   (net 30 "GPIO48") (solder_mask_margin 0.102))
  (pad "J3_17" thru_hole circle (at 11.43 10.67) (size 1.53 1.53) (drill 1.02) (layers "*.Cu" "*.Mask") (remove_unused_layers no)
   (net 31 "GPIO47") (solder_mask_margin 0.102))
  (pad "J3_18" thru_hole circle (at 11.43 13.21) (size 1.53 1.53) (drill 1.02) (layers "*.Cu" "*.Mask") (remove_unused_layers no)
   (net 32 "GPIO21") (solder_mask_margin 0.102))
  (pad "J3_19" thru_hole circle (at 11.43 15.75) (size 1.53 1.53) (drill 1.02) (layers "*.Cu" "*.Mask") (remove_unused_layers no)
   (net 33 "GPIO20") (solder_mask_margin 0.102))
  (pad "J3_20" thru_hole circle (at 11.43 18.29) (size 1.53 1.53) (drill 1.02) (layers "*.Cu" "*.Mask") (remove_unused_layers no)
   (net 34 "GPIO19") (solder_mask_margin 0.102))
  (pad "J3_21" thru_hole circle (at 11.43 20.83) (size 1.53 1.53) (drill 1.02) (layers "*.Cu" "*.Mask") (remove_unused_layers no)
   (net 10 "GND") (solder_mask_margin 0.102))
  (pad "J3_22" thru_hole circle (at 11.43 23.37) (size 1.53 1.53) (drill 1.02) (layers "*.Cu" "*.Mask") (remove_unused_layers no)
   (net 10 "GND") (solder_mask_margin 0.102)))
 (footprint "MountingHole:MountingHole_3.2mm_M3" (layer "F.Cu") (at 215.05 53.85)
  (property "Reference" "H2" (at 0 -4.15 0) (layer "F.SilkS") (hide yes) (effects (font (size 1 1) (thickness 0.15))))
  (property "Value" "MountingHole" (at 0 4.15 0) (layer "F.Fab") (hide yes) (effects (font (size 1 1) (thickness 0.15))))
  (pad "" np_thru_hole circle (at 0 0) (size 3.2 3.2) (drill 3.2) (layers "*.Cu" "*.Mask")))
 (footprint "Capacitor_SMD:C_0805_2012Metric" (layer "F.Cu") (at 234.25 84.425 -90)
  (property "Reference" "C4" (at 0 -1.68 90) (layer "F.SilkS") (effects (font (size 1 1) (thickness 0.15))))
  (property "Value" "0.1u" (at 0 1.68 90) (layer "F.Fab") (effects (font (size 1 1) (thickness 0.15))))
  (pad "1" smd roundrect (at -0.95 0 270) (size 1 1.45) (layers "F.Cu" "F.Mask" "F.Paste") (roundrect_rratio 0.25) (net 54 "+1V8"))
  (pad "2" smd roundrect (at 0.95 0 270) (size 1 1.45) (layers "F.Cu" "F.Mask" "F.Paste") (roundrect_rratio 0.25) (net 10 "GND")))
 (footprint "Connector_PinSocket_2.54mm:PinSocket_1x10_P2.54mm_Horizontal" (layer "F.Cu") (at 127.25 80.65)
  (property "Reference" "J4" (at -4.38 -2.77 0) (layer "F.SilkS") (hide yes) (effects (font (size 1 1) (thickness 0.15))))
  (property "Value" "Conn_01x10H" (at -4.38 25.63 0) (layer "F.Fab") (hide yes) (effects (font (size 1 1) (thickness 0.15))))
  (pad "1" thru_hole rect (at 0 0) (size 1.7 1.7) (drill 1) (layers "*.Cu" "*.Mask") (remove_unused_layers no) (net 1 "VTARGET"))
  (pad "2" thru_hole circle (at 0 2.54) (size 1.7 1.7) (drill 1) (layers "*.Cu" "*.Mask") (remove_unused_layers no) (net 2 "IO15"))
  (pad "3" thru_hole circle (at 0 5.08) (size 1.7 1.7) (drill 1) (layers "*.Cu" "*.Mask") (remove_unused_layers no) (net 3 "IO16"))
  (pad "4" thru_hole circle (at 0 7.62) (size 1.7 1.7) (drill 1) (layers "*.Cu" "*.Mask") (remove_unused_layers no) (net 4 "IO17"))
  (pad "5" thru_hole circle (at 0 10.16) (size 1.7 1.7) (drill 1) (layers "*.Cu" "*.Mask") (remove_unused_layers no) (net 5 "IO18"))
  (pad "6" thru_hole circle (at 0 12.7) (size 1.7 1.7) (drill 1) (layers "*.Cu" "*.Mask") (remove_unused_layers no) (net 6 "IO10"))
  (pad "7" thru_hole circle (at 0 15.24) (size 1.7 1.7) (drill 1) (layers "*.Cu" "*.Mask") (remove_unused_layers no) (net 7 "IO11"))
  (pad "8" thru_hole circle (at 0 17.78) (size 1.7 1.7) (drill 1) (layers "*.Cu" "*.Mask") (remove_unused_layers no) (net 8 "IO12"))
  (pad "9" thru_hole circle (at 0 20.32) (size 1.7 1.7) (drill 1) (layers "*.Cu" "*.Mask") (remove_unused_layers no) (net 9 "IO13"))
  (pad "10" thru_hole circle (at 0 22.86) (size 1.7 1.7) (drill 1) (layers "*.Cu" "*.Mask") (remove_unused_layers no) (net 10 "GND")))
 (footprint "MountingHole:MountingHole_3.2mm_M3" (layer "F.Cu") (at 128.55 120)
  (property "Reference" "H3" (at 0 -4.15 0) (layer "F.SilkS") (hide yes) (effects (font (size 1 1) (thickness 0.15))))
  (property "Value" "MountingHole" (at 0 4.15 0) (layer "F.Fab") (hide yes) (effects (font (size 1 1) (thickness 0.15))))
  (pad "" np_thru_hole circle (at 0 0) (size 3.2 3.2) (drill 3.2) (layers "*.Cu" "*.Mask")))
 (gr_rect (start 124.4 49.31) (end 219.7 124.16) (stroke (width 0.05) (type default)) (fill no) (layer "Edge.Cuts"))
 (segment (start 176.065 65.975) (end 176.06 65.97) (width 0.2) (layer "F.Cu") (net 17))
 (segment (start 176.065 71.055) (end 176.06 71.05) (width 0.2) (layer "F.Cu") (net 19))
 (segment (start 176.065 76.135) (end 176.06 76.13) (width 0.2) (layer "F.Cu") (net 21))
 (segment (start 176.065 81.215) (end 176.06 81.21) (width 0.2) (layer "F.Cu") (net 23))
 (segment (start 176.065 83.755) (end 176.06 83.75) (width 0.2) (layer "F.Cu") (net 24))
 (segment (start 176.065 88.835) (end 176.06 88.83) (width 0.2) (layer "F.Cu") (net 26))
 (segment (start 176.065 93.915) (end 176.06 93.91) (width 0.2) (layer "F.Cu") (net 28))
 (segment (start 176.065 98.995) (end 176.06 98.99) (width 0.2) (layer "F.Cu") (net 29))
 (segment (start 176.065 104.075) (end 176.06 104.07) (width 0.2) (layer "F.Cu") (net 31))
 (segment (start 176.065 111.695) (end 176.06 111.69) (width 0.2) (layer "F.Cu") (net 34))
 (segment (start 176.065 109.155) (end 176.06 109.15) (width 0.2) (layer "F.Cu") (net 33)))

